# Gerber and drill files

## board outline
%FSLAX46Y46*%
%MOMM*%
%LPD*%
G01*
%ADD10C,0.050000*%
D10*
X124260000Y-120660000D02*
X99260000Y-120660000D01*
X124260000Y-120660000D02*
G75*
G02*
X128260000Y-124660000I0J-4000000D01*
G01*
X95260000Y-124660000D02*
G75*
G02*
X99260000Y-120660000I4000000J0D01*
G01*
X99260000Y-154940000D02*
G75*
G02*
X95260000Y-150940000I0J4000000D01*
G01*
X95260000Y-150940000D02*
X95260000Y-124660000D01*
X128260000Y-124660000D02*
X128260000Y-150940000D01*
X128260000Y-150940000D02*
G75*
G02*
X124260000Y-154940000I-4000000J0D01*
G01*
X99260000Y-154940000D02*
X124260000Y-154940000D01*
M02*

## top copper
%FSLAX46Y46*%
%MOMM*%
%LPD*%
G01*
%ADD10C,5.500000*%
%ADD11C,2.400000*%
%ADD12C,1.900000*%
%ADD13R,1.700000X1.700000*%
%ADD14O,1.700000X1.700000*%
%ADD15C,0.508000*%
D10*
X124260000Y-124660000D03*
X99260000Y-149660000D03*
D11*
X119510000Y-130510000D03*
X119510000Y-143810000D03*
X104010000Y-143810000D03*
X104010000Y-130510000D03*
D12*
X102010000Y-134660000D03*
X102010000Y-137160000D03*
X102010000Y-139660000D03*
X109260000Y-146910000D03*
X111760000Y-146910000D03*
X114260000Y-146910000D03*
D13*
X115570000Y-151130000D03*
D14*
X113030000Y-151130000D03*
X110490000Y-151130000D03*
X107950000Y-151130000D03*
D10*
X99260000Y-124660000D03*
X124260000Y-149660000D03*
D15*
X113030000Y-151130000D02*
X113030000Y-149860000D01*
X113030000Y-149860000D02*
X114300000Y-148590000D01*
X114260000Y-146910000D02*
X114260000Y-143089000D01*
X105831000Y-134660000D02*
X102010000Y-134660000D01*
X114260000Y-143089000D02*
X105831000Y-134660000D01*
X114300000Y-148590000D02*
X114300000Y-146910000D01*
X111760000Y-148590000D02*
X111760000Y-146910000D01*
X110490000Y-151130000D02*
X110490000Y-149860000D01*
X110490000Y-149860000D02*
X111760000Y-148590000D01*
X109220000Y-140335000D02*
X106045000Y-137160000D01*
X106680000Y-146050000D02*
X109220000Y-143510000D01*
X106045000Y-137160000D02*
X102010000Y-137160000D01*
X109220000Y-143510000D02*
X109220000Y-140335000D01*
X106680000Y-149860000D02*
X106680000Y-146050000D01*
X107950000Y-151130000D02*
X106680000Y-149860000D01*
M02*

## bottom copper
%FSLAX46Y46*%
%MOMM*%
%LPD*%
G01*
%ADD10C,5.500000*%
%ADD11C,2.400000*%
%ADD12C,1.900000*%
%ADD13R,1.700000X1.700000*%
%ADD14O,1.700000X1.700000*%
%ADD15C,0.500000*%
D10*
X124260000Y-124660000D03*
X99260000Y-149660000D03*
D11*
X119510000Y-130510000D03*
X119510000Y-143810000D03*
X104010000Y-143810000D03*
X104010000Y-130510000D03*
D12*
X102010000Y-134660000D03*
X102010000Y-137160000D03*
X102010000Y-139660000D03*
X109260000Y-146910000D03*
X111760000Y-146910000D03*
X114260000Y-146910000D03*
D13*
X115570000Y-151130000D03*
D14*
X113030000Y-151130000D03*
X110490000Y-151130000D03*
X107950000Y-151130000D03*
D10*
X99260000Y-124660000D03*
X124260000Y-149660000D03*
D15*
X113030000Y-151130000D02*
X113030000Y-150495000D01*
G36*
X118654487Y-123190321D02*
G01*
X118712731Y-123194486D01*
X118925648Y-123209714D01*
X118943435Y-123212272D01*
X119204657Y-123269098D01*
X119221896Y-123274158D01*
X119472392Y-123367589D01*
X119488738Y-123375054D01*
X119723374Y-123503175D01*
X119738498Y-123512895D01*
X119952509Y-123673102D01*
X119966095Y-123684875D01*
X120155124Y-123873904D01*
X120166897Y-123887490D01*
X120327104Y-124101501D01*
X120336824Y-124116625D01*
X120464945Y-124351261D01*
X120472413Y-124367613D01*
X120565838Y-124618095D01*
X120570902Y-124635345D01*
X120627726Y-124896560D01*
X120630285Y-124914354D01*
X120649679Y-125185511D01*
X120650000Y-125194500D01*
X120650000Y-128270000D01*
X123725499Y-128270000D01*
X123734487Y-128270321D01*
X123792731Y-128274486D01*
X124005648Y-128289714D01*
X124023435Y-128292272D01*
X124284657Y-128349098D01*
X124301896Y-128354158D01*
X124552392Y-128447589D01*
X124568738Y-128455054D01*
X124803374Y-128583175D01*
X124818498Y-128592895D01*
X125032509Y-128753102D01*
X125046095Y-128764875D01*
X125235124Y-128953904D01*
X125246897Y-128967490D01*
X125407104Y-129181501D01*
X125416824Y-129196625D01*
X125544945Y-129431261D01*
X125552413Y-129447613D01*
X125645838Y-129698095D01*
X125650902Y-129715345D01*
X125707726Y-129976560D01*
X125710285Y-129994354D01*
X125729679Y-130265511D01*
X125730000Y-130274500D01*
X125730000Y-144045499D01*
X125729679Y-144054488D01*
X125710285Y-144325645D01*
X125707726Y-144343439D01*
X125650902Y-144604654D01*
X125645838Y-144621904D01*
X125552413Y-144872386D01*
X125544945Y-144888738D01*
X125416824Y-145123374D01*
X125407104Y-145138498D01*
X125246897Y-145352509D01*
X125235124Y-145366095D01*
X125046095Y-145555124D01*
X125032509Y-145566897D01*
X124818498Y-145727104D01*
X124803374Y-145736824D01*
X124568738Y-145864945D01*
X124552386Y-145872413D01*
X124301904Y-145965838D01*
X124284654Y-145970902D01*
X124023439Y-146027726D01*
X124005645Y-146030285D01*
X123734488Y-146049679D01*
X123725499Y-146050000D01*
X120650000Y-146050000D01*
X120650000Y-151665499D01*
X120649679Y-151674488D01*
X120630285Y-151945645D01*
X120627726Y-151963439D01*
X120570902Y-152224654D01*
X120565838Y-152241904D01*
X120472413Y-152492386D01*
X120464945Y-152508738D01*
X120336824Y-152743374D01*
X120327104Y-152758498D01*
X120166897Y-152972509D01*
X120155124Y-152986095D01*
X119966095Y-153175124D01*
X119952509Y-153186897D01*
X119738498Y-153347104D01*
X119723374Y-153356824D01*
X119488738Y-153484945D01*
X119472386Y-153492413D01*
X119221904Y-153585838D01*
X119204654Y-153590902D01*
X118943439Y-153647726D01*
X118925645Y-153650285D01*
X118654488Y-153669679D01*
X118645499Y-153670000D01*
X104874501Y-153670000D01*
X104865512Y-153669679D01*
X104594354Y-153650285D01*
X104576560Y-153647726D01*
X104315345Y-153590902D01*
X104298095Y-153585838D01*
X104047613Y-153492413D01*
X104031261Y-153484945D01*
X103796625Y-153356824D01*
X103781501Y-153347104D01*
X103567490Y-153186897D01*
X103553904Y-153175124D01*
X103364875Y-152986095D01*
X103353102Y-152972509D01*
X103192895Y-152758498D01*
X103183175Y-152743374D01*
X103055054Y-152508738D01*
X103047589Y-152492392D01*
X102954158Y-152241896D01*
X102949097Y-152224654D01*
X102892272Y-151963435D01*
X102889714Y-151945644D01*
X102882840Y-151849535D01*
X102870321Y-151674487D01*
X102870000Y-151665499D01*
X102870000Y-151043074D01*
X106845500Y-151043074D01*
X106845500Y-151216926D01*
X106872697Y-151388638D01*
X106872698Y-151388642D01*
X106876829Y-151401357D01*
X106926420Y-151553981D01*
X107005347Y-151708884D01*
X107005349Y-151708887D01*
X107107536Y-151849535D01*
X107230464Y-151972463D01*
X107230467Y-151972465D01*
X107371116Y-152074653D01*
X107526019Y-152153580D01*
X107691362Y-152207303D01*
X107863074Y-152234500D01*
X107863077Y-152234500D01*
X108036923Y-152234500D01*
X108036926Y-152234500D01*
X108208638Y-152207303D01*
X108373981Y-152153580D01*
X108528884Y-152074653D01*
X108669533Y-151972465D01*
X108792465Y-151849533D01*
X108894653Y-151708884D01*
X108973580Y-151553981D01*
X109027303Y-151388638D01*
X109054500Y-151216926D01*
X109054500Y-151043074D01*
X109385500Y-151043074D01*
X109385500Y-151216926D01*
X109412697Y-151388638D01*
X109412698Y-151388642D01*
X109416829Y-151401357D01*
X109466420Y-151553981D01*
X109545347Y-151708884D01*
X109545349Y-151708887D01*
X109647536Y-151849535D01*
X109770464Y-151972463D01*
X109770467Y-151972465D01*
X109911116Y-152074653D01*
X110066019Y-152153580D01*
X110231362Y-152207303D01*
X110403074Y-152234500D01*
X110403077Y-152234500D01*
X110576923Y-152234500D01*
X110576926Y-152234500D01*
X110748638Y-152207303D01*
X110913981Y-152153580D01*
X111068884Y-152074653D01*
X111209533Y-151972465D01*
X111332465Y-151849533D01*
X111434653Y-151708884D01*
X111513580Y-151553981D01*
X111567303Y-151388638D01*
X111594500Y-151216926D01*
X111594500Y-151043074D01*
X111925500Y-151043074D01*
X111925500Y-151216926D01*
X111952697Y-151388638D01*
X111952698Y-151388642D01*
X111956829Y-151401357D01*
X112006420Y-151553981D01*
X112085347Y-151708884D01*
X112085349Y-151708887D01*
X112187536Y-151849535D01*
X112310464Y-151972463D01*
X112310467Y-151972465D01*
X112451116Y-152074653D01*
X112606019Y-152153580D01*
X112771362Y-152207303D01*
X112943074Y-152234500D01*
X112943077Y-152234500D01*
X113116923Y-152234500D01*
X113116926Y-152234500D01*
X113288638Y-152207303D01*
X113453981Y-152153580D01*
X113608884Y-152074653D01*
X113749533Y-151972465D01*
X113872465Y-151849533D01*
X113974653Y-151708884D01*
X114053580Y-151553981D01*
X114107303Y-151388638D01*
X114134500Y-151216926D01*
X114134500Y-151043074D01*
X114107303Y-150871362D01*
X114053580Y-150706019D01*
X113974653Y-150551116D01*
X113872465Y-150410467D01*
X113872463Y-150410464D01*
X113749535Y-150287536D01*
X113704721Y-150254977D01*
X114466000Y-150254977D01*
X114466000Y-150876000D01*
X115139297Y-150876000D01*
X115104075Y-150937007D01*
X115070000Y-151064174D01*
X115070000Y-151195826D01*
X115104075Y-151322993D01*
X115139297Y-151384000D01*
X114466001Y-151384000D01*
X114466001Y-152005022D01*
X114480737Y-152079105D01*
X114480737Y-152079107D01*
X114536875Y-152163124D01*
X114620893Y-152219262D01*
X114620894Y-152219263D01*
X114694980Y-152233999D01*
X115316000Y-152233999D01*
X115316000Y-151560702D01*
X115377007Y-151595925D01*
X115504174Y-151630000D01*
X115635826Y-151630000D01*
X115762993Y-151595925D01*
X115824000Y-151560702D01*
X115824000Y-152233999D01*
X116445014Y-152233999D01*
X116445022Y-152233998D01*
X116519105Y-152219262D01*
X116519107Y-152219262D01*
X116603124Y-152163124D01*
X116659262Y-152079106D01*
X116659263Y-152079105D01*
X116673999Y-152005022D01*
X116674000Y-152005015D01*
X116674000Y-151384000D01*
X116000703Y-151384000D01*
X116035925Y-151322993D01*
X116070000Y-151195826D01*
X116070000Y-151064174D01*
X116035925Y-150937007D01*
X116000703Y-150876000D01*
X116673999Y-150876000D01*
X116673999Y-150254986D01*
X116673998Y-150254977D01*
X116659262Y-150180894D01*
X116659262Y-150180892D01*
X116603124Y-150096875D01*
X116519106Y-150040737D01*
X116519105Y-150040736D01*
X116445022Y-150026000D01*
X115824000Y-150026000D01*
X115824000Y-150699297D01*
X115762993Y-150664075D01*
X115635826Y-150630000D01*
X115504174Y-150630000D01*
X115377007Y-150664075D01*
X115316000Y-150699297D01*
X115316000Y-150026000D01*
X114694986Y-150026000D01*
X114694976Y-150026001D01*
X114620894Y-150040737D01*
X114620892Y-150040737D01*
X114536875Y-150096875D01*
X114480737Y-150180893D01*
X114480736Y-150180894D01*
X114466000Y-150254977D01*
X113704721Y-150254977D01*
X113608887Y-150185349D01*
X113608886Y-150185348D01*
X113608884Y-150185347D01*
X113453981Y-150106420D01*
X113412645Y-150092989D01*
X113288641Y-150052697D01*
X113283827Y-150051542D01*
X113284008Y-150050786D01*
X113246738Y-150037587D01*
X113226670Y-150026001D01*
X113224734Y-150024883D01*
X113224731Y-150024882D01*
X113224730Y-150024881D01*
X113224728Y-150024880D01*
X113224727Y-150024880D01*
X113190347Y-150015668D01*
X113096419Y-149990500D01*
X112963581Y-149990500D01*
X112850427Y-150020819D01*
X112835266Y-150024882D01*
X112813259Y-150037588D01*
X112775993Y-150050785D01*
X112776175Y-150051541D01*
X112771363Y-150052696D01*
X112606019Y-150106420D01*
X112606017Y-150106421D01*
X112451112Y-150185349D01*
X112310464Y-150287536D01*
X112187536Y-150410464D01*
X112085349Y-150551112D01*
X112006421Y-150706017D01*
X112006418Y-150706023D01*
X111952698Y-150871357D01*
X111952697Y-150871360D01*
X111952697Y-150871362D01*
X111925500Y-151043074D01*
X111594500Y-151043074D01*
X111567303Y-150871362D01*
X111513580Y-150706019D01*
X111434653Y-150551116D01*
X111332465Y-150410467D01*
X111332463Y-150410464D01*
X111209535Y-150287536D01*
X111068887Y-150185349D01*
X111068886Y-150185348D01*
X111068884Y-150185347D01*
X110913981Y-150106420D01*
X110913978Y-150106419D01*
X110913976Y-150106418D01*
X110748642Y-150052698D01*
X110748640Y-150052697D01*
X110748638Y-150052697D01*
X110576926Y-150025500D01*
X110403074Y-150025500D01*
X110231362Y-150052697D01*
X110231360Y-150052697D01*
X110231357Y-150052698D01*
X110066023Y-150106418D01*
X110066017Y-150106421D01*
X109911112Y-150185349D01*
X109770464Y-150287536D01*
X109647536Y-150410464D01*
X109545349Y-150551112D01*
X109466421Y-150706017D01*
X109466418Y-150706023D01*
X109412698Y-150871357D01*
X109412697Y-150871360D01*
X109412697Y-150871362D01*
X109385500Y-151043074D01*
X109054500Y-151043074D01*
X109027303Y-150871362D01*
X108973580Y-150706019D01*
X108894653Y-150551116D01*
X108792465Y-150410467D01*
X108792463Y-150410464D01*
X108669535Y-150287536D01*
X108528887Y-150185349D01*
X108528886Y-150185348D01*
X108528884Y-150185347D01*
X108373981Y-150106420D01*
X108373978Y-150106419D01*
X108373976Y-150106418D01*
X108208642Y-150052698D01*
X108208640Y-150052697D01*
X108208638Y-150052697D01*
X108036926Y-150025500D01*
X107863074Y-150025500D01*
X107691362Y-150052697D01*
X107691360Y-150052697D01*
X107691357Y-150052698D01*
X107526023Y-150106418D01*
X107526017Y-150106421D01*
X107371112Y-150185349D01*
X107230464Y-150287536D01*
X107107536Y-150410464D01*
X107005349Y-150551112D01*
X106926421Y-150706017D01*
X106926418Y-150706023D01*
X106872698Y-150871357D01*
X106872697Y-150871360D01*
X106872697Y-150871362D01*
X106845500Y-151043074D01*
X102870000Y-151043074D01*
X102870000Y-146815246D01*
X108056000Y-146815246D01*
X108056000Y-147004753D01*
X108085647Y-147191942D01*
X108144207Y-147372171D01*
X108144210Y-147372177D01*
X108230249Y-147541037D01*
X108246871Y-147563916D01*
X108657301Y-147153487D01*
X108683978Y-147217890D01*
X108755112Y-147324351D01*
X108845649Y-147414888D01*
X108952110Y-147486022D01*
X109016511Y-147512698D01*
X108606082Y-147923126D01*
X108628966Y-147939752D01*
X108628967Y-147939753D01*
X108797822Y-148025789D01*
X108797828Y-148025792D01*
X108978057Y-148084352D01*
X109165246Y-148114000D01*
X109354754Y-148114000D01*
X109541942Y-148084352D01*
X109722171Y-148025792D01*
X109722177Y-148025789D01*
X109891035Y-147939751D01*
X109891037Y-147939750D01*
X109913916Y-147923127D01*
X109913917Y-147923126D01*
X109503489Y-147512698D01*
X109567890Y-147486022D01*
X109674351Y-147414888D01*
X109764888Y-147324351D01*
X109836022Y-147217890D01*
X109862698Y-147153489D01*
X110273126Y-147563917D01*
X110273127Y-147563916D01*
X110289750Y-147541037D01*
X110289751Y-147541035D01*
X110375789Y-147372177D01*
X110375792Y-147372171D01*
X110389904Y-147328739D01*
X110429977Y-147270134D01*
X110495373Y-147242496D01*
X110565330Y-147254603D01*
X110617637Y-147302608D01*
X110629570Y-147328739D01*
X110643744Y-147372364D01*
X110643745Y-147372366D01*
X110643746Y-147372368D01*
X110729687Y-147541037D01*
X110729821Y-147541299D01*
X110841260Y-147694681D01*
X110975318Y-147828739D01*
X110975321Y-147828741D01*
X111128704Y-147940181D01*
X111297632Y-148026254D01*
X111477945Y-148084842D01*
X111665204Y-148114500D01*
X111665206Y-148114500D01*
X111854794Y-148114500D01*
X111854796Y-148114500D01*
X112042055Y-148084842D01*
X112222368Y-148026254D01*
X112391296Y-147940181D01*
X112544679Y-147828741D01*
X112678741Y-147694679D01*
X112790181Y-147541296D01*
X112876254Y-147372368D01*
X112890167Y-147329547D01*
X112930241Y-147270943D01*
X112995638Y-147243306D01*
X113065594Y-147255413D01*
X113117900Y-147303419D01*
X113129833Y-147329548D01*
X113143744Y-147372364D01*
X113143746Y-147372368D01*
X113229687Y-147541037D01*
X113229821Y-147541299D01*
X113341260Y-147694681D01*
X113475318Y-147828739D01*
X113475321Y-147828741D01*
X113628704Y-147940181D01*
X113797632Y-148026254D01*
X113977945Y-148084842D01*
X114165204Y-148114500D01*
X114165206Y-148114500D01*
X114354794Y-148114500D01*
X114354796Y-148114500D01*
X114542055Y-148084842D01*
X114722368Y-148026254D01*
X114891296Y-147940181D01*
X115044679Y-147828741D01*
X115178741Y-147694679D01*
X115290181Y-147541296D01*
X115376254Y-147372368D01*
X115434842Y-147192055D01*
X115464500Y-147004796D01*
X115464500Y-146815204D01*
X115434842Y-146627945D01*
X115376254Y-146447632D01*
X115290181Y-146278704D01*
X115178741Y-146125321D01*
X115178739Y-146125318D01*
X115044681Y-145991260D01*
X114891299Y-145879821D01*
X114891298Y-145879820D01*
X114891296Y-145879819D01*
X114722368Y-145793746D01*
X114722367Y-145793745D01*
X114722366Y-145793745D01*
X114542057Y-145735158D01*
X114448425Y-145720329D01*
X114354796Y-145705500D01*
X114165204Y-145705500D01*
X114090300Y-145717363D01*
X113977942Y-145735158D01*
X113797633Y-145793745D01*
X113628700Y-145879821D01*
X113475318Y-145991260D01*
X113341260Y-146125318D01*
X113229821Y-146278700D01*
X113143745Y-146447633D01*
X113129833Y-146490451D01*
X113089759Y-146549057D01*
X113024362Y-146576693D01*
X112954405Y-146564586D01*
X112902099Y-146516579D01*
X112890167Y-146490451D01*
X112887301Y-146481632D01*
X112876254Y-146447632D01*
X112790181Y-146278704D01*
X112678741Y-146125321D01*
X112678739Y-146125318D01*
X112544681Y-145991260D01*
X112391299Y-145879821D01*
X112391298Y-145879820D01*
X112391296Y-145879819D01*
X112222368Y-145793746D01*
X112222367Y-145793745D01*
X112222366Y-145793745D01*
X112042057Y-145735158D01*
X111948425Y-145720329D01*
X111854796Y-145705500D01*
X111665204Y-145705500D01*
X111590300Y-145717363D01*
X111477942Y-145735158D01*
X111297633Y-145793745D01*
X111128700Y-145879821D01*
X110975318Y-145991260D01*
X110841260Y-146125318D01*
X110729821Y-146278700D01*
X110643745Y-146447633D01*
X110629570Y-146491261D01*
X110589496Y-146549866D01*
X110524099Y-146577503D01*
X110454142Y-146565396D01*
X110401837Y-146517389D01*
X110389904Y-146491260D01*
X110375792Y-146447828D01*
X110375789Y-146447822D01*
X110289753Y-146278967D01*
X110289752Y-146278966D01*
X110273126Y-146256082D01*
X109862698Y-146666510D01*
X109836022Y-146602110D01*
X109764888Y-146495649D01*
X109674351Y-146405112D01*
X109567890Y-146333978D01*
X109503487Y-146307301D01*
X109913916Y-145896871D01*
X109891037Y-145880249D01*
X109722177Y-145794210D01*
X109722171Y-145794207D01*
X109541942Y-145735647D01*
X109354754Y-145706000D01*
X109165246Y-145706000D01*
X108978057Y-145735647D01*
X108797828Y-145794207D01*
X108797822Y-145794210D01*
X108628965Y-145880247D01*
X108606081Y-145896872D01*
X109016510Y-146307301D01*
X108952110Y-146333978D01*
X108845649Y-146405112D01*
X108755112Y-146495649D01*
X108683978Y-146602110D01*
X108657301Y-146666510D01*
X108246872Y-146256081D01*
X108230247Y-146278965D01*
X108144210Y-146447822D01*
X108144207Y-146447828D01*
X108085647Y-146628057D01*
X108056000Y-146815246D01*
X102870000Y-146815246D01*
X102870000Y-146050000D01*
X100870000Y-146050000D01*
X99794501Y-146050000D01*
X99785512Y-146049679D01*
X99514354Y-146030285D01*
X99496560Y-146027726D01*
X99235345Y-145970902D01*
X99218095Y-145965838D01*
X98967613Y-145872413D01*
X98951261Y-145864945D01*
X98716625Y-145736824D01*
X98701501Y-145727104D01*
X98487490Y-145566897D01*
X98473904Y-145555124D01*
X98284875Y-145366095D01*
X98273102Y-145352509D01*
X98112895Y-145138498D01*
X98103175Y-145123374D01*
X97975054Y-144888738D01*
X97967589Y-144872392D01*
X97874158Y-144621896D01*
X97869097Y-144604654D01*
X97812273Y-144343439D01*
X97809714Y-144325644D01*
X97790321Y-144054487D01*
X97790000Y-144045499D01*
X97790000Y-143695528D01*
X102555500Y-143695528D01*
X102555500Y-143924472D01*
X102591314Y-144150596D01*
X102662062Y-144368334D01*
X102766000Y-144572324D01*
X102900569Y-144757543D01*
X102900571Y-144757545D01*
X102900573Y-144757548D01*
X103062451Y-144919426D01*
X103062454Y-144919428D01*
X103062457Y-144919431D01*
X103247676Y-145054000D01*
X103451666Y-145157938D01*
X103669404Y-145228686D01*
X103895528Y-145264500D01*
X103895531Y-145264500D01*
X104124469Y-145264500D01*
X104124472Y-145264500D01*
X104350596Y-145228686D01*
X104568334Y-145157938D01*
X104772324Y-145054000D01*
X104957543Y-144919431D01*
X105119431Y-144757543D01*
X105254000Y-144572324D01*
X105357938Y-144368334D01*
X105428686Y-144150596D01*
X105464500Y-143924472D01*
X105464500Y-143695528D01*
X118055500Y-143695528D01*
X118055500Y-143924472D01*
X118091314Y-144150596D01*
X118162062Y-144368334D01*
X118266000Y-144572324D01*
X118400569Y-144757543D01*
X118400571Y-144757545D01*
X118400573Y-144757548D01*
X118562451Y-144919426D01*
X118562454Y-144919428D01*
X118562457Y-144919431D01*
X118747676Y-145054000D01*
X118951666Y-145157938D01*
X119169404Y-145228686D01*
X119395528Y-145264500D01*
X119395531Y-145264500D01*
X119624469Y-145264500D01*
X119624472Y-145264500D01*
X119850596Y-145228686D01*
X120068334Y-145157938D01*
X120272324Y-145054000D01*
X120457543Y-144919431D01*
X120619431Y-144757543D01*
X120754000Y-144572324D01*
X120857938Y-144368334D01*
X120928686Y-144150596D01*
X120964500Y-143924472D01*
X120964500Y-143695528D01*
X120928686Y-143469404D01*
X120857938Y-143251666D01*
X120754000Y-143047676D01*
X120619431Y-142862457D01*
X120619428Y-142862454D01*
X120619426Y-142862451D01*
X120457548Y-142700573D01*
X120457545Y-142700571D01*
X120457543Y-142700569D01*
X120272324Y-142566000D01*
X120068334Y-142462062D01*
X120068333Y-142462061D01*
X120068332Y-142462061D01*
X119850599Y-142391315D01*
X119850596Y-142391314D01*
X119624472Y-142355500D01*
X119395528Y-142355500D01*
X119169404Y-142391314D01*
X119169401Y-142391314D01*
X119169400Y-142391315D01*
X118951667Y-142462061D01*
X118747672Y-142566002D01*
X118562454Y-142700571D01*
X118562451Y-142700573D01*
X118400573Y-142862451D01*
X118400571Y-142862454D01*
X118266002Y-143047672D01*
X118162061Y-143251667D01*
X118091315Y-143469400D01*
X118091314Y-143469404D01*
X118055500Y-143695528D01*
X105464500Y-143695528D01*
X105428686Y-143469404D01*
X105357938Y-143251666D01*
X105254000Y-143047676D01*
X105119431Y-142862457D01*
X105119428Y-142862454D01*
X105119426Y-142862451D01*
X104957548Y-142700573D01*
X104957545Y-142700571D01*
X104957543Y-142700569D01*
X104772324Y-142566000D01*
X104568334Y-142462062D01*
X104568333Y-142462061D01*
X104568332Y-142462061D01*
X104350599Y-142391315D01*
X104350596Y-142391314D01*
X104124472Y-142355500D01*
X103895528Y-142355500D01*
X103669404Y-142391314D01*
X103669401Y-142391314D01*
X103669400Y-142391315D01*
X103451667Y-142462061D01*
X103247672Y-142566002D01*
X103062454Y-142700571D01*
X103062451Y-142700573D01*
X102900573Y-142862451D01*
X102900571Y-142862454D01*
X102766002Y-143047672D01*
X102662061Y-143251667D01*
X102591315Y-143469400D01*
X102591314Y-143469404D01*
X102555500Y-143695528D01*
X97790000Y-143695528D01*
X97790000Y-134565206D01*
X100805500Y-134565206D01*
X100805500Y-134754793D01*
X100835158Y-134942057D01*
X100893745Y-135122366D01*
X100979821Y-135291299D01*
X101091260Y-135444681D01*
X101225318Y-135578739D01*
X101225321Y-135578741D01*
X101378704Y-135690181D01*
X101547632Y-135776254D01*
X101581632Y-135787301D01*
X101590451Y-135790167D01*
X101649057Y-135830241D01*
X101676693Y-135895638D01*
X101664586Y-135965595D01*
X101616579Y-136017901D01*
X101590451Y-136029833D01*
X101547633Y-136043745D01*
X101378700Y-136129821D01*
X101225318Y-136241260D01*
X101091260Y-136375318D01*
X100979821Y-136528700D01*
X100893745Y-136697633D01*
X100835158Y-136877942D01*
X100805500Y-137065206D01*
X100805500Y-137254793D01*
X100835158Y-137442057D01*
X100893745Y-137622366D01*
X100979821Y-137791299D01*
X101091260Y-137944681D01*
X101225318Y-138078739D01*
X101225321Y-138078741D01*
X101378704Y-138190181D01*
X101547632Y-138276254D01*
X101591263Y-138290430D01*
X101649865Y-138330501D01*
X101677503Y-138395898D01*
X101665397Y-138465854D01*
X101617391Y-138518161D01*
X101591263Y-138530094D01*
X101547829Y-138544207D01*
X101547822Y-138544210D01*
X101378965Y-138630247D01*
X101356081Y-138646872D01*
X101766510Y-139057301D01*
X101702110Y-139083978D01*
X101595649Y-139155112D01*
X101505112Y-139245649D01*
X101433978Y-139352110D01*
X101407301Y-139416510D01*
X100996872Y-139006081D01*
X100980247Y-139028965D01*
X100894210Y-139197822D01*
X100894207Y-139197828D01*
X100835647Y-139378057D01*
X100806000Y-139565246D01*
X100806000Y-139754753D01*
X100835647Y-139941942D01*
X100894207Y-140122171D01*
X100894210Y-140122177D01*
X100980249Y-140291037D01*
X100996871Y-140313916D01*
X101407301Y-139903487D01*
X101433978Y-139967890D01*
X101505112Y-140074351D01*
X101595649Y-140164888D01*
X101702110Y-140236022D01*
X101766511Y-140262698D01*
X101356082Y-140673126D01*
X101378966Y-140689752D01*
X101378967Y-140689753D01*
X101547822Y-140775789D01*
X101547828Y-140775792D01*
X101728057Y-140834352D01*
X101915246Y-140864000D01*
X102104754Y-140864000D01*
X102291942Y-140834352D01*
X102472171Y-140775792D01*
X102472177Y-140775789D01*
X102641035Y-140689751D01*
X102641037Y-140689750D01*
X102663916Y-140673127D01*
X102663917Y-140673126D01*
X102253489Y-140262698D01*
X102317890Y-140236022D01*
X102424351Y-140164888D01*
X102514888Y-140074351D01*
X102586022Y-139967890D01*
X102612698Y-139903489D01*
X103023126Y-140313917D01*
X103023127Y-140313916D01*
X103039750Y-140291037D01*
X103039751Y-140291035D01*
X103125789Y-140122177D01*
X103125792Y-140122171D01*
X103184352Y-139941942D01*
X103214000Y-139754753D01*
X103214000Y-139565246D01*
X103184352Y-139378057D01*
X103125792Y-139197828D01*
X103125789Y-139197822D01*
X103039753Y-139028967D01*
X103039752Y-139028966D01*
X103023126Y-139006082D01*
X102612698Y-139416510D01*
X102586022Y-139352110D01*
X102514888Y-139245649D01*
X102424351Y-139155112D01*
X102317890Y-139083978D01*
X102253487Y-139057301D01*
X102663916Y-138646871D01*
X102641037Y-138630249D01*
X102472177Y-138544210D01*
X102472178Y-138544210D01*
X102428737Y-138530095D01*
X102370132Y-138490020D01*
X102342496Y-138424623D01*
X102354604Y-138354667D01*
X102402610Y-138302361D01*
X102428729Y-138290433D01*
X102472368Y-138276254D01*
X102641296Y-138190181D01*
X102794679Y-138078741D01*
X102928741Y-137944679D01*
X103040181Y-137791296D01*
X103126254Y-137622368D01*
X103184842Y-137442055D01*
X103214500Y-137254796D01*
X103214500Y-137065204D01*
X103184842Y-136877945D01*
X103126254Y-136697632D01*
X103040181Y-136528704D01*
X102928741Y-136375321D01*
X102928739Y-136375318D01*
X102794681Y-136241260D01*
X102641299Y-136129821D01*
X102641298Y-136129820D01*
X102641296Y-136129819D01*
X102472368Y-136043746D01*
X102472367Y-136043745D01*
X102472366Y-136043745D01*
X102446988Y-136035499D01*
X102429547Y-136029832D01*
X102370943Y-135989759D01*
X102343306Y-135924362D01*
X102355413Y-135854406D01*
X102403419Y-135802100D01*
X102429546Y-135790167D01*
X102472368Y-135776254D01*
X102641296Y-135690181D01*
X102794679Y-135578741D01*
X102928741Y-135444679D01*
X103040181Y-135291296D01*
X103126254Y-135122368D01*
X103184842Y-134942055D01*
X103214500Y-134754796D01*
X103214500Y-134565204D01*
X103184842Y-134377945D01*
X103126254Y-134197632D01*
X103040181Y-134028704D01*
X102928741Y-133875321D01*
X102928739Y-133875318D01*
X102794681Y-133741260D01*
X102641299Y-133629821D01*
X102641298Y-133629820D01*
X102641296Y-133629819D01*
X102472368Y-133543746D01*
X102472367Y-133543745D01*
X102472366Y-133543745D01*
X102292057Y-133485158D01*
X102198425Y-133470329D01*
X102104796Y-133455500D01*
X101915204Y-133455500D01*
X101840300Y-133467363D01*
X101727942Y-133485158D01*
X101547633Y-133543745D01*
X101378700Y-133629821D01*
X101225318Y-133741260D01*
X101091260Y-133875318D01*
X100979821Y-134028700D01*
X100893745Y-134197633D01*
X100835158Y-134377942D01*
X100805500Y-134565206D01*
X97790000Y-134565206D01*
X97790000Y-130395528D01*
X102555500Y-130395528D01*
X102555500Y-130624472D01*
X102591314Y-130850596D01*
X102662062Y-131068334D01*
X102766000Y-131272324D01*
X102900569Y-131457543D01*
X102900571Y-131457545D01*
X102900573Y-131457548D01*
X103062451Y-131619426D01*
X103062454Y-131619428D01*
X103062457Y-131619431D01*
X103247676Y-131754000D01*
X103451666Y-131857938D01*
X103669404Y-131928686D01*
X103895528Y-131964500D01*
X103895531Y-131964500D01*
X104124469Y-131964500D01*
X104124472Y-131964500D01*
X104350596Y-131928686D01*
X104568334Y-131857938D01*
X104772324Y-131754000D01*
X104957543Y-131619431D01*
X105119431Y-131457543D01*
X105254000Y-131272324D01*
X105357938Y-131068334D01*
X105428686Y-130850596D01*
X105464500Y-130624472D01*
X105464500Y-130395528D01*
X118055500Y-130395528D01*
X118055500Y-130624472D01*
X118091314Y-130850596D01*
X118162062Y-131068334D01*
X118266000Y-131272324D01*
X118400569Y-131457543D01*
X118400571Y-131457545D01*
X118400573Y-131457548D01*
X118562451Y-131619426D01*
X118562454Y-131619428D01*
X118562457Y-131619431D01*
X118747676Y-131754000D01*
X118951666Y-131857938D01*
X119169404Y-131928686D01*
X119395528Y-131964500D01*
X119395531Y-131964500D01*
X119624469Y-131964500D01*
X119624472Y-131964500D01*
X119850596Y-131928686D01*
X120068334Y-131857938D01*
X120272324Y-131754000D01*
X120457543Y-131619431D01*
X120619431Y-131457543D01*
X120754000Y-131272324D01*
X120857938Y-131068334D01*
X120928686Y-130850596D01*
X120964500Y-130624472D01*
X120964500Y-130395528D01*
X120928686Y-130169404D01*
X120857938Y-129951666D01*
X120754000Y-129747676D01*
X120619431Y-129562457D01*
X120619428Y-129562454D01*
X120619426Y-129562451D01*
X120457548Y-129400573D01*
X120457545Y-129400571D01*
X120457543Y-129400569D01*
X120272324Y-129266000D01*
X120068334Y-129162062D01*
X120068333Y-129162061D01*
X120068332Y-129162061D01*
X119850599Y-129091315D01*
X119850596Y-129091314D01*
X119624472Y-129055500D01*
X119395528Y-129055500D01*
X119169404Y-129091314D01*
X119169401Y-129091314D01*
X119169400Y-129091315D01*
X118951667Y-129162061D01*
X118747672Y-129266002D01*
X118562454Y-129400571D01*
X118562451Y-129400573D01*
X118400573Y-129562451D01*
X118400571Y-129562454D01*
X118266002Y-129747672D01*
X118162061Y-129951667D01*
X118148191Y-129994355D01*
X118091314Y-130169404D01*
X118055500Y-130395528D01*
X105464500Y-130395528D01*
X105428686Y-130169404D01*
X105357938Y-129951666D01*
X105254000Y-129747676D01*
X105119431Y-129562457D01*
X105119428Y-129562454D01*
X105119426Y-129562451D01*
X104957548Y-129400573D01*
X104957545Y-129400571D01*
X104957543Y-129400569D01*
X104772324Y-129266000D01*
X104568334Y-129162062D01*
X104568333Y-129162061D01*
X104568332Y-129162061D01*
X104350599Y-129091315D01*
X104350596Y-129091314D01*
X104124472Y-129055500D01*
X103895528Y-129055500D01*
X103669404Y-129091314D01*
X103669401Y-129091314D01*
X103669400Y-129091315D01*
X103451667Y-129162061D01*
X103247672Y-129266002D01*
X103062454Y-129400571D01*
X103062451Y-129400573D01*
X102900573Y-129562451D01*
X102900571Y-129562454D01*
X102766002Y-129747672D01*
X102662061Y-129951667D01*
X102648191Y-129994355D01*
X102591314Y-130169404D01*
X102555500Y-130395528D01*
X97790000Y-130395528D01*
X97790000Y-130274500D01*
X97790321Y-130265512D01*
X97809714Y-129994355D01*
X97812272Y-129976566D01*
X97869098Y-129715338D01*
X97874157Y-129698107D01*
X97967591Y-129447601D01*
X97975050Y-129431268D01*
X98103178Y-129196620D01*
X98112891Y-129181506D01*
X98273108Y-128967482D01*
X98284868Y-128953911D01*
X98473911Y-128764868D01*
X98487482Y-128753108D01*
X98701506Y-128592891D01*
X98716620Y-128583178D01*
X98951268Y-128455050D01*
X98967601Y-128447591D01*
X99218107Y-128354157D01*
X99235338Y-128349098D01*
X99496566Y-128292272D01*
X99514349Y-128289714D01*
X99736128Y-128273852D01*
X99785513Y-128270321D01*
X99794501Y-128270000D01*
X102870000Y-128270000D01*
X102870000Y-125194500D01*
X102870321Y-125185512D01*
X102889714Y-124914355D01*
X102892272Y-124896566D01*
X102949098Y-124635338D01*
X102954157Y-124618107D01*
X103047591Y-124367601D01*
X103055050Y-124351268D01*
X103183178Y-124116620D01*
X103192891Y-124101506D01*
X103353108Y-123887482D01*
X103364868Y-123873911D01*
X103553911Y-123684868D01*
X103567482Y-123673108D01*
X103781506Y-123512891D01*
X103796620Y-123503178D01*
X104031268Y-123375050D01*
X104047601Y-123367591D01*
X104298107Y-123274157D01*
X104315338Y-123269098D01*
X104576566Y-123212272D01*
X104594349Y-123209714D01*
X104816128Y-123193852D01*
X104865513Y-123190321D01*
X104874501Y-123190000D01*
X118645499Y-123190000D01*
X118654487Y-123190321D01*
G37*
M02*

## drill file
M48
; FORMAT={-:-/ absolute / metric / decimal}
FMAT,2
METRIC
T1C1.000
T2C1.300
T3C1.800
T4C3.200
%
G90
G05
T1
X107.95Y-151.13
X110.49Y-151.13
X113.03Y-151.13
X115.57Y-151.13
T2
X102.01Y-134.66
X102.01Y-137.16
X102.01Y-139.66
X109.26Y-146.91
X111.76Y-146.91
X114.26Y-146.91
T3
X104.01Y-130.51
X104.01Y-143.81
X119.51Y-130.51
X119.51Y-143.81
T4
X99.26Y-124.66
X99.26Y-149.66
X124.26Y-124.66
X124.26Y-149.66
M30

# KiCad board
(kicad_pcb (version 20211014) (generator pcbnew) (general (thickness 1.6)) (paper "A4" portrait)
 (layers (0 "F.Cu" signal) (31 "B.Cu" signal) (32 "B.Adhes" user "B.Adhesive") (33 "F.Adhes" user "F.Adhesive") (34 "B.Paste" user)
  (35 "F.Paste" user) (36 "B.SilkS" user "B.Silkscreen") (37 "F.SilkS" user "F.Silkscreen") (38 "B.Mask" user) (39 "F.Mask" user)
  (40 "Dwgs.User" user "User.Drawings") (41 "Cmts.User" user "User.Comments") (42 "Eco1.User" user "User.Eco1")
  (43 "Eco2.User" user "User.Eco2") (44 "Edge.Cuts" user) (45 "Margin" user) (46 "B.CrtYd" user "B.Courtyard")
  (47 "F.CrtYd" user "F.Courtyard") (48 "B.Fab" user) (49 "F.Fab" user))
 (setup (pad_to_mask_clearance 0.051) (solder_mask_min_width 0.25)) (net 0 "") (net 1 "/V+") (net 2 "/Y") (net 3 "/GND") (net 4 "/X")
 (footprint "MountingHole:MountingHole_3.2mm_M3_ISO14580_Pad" (layer "F.Cu") (at 124.26 124.66)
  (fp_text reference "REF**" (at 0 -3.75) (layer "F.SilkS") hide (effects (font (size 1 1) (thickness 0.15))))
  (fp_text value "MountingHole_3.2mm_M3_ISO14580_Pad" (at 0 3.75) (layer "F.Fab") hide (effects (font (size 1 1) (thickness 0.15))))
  (pad "1" thru_hole circle locked (at 0 0) (size 5.5 5.5) (drill 3.2) (layers *.Cu *.Mask)))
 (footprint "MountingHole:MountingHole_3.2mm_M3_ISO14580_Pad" (layer "F.Cu") (at 99.26 149.66)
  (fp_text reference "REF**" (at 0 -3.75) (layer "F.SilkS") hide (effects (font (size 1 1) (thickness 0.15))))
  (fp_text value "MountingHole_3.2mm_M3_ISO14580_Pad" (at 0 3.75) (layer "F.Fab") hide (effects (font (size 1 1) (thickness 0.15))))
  (pad "1" thru_hole circle locked (at 0 0) (size 5.5 5.5) (drill 3.2) (layers *.Cu *.Mask)))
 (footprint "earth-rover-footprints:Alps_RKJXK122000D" (layer "F.Cu") (at 111.76 137.16 180)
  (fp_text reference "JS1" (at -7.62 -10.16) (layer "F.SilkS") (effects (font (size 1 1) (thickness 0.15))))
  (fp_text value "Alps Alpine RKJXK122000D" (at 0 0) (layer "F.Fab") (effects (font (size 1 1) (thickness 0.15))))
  (pad "" thru_hole circle locked (at -7.75 6.65 180) (size 2.4 2.4) (drill 1.8) (layers *.Cu *.Mask))
  (pad "" thru_hole circle locked (at -7.75 -6.65 180) (size 2.4 2.4) (drill 1.8) (layers *.Cu *.Mask))
  (pad "" thru_hole circle locked (at 7.75 -6.65 180) (size 2.4 2.4) (drill 1.8) (layers *.Cu *.Mask))
  (pad "" thru_hole circle locked (at 7.75 6.65 180) (size 2.4 2.4) (drill 1.8) (layers *.Cu *.Mask))
  (pad "1" thru_hole circle locked (at 9.75 2.5 180) (size 1.9 1.9) (drill 1.3) (layers *.Cu *.Mask) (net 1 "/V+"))
  (pad "2" thru_hole circle locked (at 9.75 0 180) (size 1.9 1.9) (drill 1.3) (layers *.Cu *.Mask) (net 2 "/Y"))
  (pad "3" thru_hole circle locked (at 9.75 -2.5 180) (size 1.9 1.9) (drill 1.3) (layers *.Cu *.Mask) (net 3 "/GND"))
  (pad "4" thru_hole circle locked (at 2.5 -9.75 180) (size 1.9 1.9) (drill 1.3) (layers *.Cu *.Mask) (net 3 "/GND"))
  (pad "5" thru_hole circle locked (at 0 -9.75 180) (size 1.9 1.9) (drill 1.3) (layers *.Cu *.Mask) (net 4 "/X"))
  (pad "6" thru_hole circle locked (at -2.5 -9.75 180) (size 1.9 1.9) (drill 1.3) (layers *.Cu *.Mask) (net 1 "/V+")))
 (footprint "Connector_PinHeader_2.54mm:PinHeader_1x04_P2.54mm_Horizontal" (layer "F.Cu") (at 115.57 151.13 -90)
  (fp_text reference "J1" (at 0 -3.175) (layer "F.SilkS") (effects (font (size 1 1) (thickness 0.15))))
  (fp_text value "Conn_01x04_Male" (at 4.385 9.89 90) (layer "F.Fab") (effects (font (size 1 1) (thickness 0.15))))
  (pad "1" thru_hole rect locked (at 0 0 270) (size 1.7 1.7) (drill 1) (layers *.Cu *.Mask) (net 3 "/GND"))
  (pad "2" thru_hole oval locked (at 0 2.54 270) (size 1.7 1.7) (drill 1) (layers *.Cu *.Mask) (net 1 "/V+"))
  (pad "3" thru_hole oval locked (at 0 5.08 270) (size 1.7 1.7) (drill 1) (layers *.Cu *.Mask) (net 4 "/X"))
  (pad "4" thru_hole oval locked (at 0 7.62 270) (size 1.7 1.7) (drill 1) (layers *.Cu *.Mask) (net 2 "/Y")))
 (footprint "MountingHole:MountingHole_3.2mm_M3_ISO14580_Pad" (layer "F.Cu") (at 99.26 124.66)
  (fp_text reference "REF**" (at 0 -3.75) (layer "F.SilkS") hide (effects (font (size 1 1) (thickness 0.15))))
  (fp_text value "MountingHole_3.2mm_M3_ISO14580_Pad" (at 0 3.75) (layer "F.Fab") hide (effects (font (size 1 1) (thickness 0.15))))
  (pad "1" thru_hole circle locked (at 0 0) (size 5.5 5.5) (drill 3.2) (layers *.Cu *.Mask)))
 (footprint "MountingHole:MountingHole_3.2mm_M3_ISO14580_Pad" (layer "F.Cu") (at 124.26 149.66)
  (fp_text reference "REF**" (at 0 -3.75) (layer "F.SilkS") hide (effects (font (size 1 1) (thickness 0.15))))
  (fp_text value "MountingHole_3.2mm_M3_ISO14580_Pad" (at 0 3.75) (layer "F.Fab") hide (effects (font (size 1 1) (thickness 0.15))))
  (pad "1" thru_hole circle locked (at 0 0) (size 5.5 5.5) (drill 3.2) (layers *.Cu *.Mask)))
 (gr_line (start 124.26 120.66) (end 99.26 120.66) (layer "Edge.Cuts") (width 0.05))
 (gr_arc (start 124.26 120.66) (mid 127.088427 121.831573) (end 128.26 124.66) (layer "Edge.Cuts") (width 0.05))
 (gr_arc (start 95.26 124.66) (mid 96.431573 121.831573) (end 99.26 120.66) (layer "Edge.Cuts") (width 0.05))
 (gr_arc (start 99.26 154.94) (mid 96.431573 153.768427) (end 95.26 150.94) (layer "Edge.Cuts") (width 0.05))
 (gr_line (start 95.26 150.94) (end 95.26 124.66) (layer "Edge.Cuts") (width 0.05))
 (gr_line (start 128.26 124.66) (end 128.26 150.94) (layer "Edge.Cuts") (width 0.05))
 (gr_arc (start 128.26 150.94) (mid 127.088427 153.768427) (end 124.26 154.94) (layer "Edge.Cuts") (width 0.05))
 (gr_line (start 99.26 154.94) (end 124.26 154.94) (layer "Edge.Cuts") (width 0.05))
 (segment (start 113.03 151.13) (end 113.03 149.86) (width 0.508) (layer "F.Cu") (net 1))
 (segment (start 113.03 149.86) (end 114.3 148.59) (width 0.508) (layer "F.Cu") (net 1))
 (segment (start 114.26 146.91) (end 114.26 143.089) (width 0.508) (layer "F.Cu") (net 1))
 (segment (start 105.831 134.66) (end 102.01 134.66) (width 0.508) (layer "F.Cu") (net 1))
 (segment (start 114.26 143.089) (end 105.831 134.66) (width 0.508) (layer "F.Cu") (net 1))
 (segment (start 114.3 148.59) (end 114.3 146.91) (width 0.508) (layer "F.Cu") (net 1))
 (segment (start 113.03 151.13) (end 113.03 150.495) (width 0.5) (layer "B.Cu") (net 1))
 (segment (start 111.76 148.59) (end 111.76 146.91) (width 0.508) (layer "F.Cu") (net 4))
 (segment (start 110.49 151.13) (end 110.49 149.86) (width 0.508) (layer "F.Cu") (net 4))
 (segment (start 110.49 149.86) (end 111.76 148.59) (width 0.508) (layer "F.Cu") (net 4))
 (segment (start 109.22 140.335) (end 106.045 137.16) (width 0.508) (layer "F.Cu") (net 2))
 (segment (start 106.68 146.05) (end 109.22 143.51) (width 0.508) (layer "F.Cu") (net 2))
 (segment (start 106.045 137.16) (end 102.01 137.16) (width 0.508) (layer "F.Cu") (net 2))
 (segment (start 109.22 143.51) (end 109.22 140.335) (width 0.508) (layer "F.Cu") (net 2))
 (segment (start 106.68 149.86) (end 106.68 146.05) (width 0.508) (layer "F.Cu") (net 2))
 (segment (start 107.95 151.13) (end 106.68 149.86) (width 0.508) (layer "F.Cu") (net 2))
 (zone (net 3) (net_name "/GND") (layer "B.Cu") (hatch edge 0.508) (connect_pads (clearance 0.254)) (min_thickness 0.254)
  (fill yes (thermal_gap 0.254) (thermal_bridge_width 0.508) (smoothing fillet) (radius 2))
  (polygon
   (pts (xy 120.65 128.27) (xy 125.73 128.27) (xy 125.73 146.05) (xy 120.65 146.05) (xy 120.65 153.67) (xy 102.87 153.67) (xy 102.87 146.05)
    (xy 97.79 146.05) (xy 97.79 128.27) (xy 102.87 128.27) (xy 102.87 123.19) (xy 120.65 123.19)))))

